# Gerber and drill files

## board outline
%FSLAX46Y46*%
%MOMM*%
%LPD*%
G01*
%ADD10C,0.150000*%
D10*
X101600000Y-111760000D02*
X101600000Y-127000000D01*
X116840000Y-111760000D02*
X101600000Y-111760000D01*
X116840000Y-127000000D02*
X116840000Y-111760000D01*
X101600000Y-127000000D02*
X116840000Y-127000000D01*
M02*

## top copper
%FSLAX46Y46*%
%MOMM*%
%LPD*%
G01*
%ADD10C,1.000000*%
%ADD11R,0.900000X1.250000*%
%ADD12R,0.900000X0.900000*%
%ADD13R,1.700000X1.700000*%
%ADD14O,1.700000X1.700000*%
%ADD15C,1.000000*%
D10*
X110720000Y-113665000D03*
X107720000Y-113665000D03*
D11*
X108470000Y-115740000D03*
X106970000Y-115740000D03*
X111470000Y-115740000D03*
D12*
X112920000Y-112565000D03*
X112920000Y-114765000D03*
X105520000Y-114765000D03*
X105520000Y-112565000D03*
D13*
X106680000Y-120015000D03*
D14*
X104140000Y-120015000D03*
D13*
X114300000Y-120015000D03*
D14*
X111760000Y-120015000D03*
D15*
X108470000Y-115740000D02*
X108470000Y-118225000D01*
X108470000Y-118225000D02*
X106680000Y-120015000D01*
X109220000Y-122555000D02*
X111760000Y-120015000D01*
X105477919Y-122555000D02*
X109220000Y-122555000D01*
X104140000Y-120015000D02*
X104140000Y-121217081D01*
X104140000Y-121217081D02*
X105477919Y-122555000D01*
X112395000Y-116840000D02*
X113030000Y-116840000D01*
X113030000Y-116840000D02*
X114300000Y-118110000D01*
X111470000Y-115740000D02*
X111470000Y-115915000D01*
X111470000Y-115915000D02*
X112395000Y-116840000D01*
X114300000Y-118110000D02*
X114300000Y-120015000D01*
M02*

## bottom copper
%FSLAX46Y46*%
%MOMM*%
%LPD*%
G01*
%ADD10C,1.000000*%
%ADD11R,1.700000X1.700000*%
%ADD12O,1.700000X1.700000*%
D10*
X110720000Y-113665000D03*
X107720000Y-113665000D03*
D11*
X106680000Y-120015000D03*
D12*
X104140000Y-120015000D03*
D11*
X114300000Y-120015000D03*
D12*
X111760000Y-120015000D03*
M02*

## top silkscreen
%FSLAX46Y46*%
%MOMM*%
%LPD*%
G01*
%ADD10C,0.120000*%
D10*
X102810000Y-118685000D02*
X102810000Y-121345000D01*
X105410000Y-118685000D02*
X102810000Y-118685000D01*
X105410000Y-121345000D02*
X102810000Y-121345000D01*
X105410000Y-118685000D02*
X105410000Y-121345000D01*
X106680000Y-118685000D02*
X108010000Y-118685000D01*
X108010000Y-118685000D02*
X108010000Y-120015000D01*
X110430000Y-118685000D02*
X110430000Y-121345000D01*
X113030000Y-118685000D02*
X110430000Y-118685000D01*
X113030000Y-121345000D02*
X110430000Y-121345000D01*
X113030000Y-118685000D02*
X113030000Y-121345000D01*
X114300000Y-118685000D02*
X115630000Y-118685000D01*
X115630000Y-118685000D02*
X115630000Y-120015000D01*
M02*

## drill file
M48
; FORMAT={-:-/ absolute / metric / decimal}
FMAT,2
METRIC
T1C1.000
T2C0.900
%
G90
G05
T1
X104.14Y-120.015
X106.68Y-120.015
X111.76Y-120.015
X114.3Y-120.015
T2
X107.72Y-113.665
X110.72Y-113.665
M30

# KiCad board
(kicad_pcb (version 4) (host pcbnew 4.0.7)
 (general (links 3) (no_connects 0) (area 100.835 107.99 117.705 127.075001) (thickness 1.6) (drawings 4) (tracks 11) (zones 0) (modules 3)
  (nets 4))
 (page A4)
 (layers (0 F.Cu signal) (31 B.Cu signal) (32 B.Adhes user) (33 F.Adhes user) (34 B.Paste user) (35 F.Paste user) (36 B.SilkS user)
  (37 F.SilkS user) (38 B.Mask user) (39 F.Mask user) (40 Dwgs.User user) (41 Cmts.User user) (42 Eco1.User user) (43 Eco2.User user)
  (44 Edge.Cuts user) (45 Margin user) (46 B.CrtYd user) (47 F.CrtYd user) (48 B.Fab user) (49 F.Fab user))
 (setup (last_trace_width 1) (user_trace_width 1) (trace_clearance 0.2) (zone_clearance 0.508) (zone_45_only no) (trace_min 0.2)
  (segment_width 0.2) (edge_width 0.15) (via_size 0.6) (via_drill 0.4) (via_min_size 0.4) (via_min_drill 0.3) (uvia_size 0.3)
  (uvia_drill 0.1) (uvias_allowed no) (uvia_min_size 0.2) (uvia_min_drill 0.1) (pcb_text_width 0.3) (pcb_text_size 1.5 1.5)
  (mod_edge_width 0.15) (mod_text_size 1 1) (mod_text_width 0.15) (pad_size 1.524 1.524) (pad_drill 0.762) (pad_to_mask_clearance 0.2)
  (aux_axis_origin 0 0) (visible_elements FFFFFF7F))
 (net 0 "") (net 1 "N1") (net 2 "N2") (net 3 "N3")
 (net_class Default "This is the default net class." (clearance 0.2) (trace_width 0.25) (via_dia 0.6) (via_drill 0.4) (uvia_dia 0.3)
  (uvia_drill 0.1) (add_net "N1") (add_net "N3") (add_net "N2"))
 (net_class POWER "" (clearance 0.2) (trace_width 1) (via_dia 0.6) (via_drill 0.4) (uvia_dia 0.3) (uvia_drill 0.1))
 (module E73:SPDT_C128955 (layer F.Cu) (at 109.22 113.665)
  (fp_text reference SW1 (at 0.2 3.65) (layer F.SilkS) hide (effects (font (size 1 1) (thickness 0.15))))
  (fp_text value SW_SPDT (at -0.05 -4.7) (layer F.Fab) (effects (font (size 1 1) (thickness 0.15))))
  (pad "" np_thru_hole circle (at 1.5 0) (size 1 1) (drill 0.9) (layers *.Cu *.Mask))
  (pad "" np_thru_hole circle (at -1.5 0) (size 1 1) (drill 0.9) (layers *.Cu *.Mask))
  (pad 2 smd rect (at -0.75 2.075) (size 0.9 1.25) (layers F.Cu F.Paste F.Mask) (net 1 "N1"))
  (pad 3 smd rect (at -2.25 2.075) (size 0.9 1.25) (layers F.Cu F.Paste F.Mask))
  (pad 1 smd rect (at 2.25 2.075) (size 0.9 1.25) (layers F.Cu F.Paste F.Mask) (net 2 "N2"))
  (pad 0 smd rect (at 3.7 -1.1) (size 0.9 0.9) (layers F.Cu F.Paste F.Mask))
  (pad 0 smd rect (at 3.7 1.1) (size 0.9 0.9) (layers F.Cu F.Paste F.Mask))
  (pad 0 smd rect (at -3.7 1.1) (size 0.9 0.9) (layers F.Cu F.Paste F.Mask))
  (pad 0 smd rect (at -3.7 -1.1) (size 0.9 0.9) (layers F.Cu F.Paste F.Mask)))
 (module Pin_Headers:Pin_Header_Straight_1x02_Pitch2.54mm (layer F.Cu) (at 106.68 120.015 270)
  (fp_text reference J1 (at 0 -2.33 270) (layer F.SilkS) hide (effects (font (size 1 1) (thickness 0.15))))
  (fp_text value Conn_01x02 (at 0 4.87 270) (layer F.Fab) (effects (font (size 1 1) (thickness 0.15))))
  (fp_line (start -1.33 3.87) (end 1.33 3.87) (layer F.SilkS) (width 0.12))
  (fp_line (start -1.33 1.27) (end -1.33 3.87) (layer F.SilkS) (width 0.12))
  (fp_line (start 1.33 1.27) (end 1.33 3.87) (layer F.SilkS) (width 0.12))
  (fp_line (start -1.33 1.27) (end 1.33 1.27) (layer F.SilkS) (width 0.12))
  (fp_line (start -1.33 0) (end -1.33 -1.33) (layer F.SilkS) (width 0.12))
  (fp_line (start -1.33 -1.33) (end 0 -1.33) (layer F.SilkS) (width 0.12))
  (pad 1 thru_hole rect (at 0 0 270) (size 1.7 1.7) (drill 1) (layers *.Cu *.Mask) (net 1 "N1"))
  (pad 2 thru_hole oval (at 0 2.54 270) (size 1.7 1.7) (drill 1) (layers *.Cu *.Mask) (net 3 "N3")))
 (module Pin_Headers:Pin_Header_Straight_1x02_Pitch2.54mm (layer F.Cu) (at 114.3 120.015 270)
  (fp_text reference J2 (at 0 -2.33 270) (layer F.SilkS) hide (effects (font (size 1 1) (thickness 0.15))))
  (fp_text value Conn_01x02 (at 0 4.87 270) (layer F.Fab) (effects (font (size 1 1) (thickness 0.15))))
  (fp_line (start -1.33 3.87) (end 1.33 3.87) (layer F.SilkS) (width 0.12))
  (fp_line (start -1.33 1.27) (end -1.33 3.87) (layer F.SilkS) (width 0.12))
  (fp_line (start 1.33 1.27) (end 1.33 3.87) (layer F.SilkS) (width 0.12))
  (fp_line (start -1.33 1.27) (end 1.33 1.27) (layer F.SilkS) (width 0.12))
  (fp_line (start -1.33 0) (end -1.33 -1.33) (layer F.SilkS) (width 0.12))
  (fp_line (start -1.33 -1.33) (end 0 -1.33) (layer F.SilkS) (width 0.12))
  (pad 1 thru_hole rect (at 0 0 270) (size 1.7 1.7) (drill 1) (layers *.Cu *.Mask) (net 2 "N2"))
  (pad 2 thru_hole oval (at 0 2.54 270) (size 1.7 1.7) (drill 1) (layers *.Cu *.Mask) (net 3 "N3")))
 (gr_line (start 101.6 111.76) (end 101.6 127) (layer Edge.Cuts) (width 0.15))
 (gr_line (start 116.84 111.76) (end 101.6 111.76) (layer Edge.Cuts) (width 0.15))
 (gr_line (start 116.84 127) (end 116.84 111.76) (layer Edge.Cuts) (width 0.15))
 (gr_line (start 101.6 127) (end 116.84 127) (layer Edge.Cuts) (width 0.15))
 (segment (start 108.47 115.74) (end 108.47 118.225) (width 1) (layer F.Cu) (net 1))
 (segment (start 108.47 118.225) (end 106.68 120.015) (width 1) (layer F.Cu) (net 1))
 (segment (start 109.22 122.555) (end 111.76 120.015) (width 1) (layer F.Cu) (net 3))
 (segment (start 105.477919 122.555) (end 109.22 122.555) (width 1) (layer F.Cu) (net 3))
 (segment (start 104.14 120.015) (end 104.14 121.217081) (width 1) (layer F.Cu) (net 3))
 (segment (start 104.14 121.217081) (end 105.477919 122.555) (width 1) (layer F.Cu) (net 3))
 (segment (start 112.395 116.84) (end 113.03 116.84) (width 1) (layer F.Cu) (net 2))
 (segment (start 113.03 116.84) (end 114.3 118.11) (width 1) (layer F.Cu) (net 2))
 (segment (start 111.47 115.74) (end 111.47 115.915) (width 1) (layer F.Cu) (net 2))
 (segment (start 111.47 115.915) (end 112.395 116.84) (width 1) (layer F.Cu) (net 2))
 (segment (start 114.3 118.11) (end 114.3 120.015) (width 1) (layer F.Cu) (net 2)))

